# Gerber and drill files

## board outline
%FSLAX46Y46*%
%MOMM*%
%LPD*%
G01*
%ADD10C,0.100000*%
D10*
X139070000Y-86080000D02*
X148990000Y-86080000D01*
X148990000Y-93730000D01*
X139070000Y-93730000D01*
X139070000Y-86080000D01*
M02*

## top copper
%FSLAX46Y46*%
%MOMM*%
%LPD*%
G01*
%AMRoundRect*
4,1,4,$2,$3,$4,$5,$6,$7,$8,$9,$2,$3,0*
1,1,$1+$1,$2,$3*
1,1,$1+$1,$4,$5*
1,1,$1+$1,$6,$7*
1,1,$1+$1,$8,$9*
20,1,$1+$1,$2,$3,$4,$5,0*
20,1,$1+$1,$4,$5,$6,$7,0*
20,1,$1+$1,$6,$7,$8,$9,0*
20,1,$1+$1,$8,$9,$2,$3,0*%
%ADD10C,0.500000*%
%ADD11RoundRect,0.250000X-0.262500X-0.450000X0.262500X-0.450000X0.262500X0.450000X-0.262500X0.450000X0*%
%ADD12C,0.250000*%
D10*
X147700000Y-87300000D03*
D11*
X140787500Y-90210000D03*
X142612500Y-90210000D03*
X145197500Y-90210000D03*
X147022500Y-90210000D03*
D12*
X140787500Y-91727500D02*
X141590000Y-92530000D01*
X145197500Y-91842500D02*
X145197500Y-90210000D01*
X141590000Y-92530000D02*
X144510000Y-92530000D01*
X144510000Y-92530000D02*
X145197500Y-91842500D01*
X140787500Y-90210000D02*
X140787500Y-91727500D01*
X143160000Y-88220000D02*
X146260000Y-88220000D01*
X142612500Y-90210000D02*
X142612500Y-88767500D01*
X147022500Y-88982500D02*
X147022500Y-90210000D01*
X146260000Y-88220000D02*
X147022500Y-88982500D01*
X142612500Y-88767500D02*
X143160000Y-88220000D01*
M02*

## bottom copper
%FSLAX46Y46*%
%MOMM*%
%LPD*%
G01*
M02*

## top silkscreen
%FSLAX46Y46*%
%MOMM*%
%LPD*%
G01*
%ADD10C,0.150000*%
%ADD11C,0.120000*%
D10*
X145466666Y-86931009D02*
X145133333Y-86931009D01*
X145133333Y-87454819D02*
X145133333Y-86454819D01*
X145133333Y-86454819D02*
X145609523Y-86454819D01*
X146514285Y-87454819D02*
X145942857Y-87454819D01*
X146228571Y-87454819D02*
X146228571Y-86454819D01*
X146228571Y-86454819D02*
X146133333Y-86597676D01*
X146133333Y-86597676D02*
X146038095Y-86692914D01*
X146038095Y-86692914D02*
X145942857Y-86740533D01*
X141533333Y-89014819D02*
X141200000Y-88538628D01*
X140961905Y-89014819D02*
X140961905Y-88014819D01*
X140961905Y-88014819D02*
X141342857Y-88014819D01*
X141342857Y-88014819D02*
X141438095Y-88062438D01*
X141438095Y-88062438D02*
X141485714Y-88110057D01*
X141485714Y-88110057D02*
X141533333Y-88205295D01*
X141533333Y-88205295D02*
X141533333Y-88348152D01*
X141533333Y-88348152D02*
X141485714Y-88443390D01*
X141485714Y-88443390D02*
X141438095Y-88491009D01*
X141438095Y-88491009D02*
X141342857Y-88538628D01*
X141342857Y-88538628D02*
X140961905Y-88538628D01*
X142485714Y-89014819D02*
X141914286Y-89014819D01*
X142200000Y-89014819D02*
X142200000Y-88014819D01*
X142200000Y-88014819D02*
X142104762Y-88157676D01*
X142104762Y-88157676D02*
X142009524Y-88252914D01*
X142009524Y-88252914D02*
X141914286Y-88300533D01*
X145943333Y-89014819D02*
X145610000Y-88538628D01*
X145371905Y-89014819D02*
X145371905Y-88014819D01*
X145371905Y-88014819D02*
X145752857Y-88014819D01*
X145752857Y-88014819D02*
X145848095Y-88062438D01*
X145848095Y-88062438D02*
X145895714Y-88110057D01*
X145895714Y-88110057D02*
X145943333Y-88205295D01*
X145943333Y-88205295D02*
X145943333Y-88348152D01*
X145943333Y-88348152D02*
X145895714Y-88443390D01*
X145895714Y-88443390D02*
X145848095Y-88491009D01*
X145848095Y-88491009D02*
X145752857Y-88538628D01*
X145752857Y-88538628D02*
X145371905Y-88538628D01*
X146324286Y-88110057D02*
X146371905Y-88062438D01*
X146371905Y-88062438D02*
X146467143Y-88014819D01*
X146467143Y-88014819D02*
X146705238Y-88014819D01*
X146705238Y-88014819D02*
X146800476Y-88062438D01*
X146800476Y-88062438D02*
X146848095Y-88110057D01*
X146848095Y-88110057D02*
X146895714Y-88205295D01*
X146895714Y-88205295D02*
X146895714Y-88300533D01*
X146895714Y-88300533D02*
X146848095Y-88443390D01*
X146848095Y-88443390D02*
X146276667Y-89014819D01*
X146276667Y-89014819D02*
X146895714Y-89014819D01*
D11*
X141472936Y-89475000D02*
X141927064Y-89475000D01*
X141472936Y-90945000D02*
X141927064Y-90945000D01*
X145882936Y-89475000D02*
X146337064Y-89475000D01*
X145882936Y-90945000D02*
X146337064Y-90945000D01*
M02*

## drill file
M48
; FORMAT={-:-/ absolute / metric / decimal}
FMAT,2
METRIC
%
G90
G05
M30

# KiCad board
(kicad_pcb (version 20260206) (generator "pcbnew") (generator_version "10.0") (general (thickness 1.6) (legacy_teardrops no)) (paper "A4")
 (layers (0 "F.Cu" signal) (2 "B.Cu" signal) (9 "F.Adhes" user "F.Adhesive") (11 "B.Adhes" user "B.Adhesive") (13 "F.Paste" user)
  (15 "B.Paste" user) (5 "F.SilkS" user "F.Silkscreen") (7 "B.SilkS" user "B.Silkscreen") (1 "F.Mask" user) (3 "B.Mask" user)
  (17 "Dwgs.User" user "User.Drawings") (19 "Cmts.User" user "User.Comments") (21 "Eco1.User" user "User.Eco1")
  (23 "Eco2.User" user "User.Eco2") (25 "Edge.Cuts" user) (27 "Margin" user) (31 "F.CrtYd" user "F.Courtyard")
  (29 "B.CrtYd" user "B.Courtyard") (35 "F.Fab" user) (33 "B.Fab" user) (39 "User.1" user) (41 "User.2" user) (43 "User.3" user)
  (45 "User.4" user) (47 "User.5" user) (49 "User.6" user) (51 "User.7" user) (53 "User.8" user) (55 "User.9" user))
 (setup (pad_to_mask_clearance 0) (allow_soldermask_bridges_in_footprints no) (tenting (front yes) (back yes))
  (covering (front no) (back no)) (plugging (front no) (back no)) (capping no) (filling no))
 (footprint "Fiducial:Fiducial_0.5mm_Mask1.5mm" (layer "F.Cu") (at 147.7 87.3)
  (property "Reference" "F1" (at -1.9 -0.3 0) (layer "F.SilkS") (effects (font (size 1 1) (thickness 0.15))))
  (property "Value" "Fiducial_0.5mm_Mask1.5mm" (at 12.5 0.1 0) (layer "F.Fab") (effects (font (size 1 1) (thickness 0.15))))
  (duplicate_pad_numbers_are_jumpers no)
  (pad "" smd circle (at 0 0) (size 0.5 0.5) (layers "F.Cu" "F.Mask") (solder_mask_margin 0.5) (clearance 0.5)))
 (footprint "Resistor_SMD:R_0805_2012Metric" (layer "F.Cu") (at 141.7 90.21)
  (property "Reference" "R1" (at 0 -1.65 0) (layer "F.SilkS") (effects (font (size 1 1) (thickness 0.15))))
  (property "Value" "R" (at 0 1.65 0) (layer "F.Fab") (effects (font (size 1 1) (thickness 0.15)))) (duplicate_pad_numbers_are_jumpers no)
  (fp_line (start -0.227064 -0.735) (end 0.227064 -0.735) (stroke (width 0.12) (type solid)) (layer "F.SilkS"))
  (fp_line (start -0.227064 0.735) (end 0.227064 0.735) (stroke (width 0.12) (type solid)) (layer "F.SilkS"))
  (pad "1" smd roundrect (at -0.9125 0) (size 1.025 1.4) (layers "F.Cu" "F.Mask" "F.Paste") (roundrect_rratio 0.243902)
   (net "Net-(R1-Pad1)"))
  (pad "2" smd roundrect (at 0.9125 0) (size 1.025 1.4) (layers "F.Cu" "F.Mask" "F.Paste") (roundrect_rratio 0.243902) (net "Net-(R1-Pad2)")))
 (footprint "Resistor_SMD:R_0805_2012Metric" (layer "F.Cu") (at 146.11 90.21)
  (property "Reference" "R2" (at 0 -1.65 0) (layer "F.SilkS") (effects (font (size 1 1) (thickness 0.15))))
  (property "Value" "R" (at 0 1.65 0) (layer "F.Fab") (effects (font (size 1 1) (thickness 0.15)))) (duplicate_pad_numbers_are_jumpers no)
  (fp_line (start -0.227064 -0.735) (end 0.227064 -0.735) (stroke (width 0.12) (type solid)) (layer "F.SilkS"))
  (fp_line (start -0.227064 0.735) (end 0.227064 0.735) (stroke (width 0.12) (type solid)) (layer "F.SilkS"))
  (pad "1" smd roundrect (at -0.9125 0) (size 1.025 1.4) (layers "F.Cu" "F.Mask" "F.Paste") (roundrect_rratio 0.243902)
   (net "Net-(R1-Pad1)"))
  (pad "2" smd roundrect (at 0.9125 0) (size 1.025 1.4) (layers "F.Cu" "F.Mask" "F.Paste") (roundrect_rratio 0.243902) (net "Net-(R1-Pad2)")))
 (gr_rect (start 139.07 86.08) (end 148.99 93.73) (stroke (width 0.1) (type solid)) (fill no) (layer "Edge.Cuts"))
 (segment (start 140.7875 91.7275) (end 141.59 92.53) (width 0.25) (layer "F.Cu") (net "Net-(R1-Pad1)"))
 (segment (start 145.1975 91.8425) (end 145.1975 90.21) (width 0.25) (layer "F.Cu") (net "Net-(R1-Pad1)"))
 (segment (start 141.59 92.53) (end 144.51 92.53) (width 0.25) (layer "F.Cu") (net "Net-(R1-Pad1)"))
 (segment (start 144.51 92.53) (end 145.1975 91.8425) (width 0.25) (layer "F.Cu") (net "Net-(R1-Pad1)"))
 (segment (start 140.7875 90.21) (end 140.7875 91.7275) (width 0.25) (layer "F.Cu") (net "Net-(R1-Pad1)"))
 (segment (start 143.16 88.22) (end 146.26 88.22) (width 0.25) (layer "F.Cu") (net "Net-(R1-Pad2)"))
 (segment (start 142.6125 90.21) (end 142.6125 88.7675) (width 0.25) (layer "F.Cu") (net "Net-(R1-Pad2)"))
 (segment (start 147.0225 88.9825) (end 147.0225 90.21) (width 0.25) (layer "F.Cu") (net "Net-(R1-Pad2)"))
 (segment (start 146.26 88.22) (end 147.0225 88.9825) (width 0.25) (layer "F.Cu") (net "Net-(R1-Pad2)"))
 (segment (start 142.6125 88.7675) (end 143.16 88.22) (width 0.25) (layer "F.Cu") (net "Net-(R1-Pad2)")))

